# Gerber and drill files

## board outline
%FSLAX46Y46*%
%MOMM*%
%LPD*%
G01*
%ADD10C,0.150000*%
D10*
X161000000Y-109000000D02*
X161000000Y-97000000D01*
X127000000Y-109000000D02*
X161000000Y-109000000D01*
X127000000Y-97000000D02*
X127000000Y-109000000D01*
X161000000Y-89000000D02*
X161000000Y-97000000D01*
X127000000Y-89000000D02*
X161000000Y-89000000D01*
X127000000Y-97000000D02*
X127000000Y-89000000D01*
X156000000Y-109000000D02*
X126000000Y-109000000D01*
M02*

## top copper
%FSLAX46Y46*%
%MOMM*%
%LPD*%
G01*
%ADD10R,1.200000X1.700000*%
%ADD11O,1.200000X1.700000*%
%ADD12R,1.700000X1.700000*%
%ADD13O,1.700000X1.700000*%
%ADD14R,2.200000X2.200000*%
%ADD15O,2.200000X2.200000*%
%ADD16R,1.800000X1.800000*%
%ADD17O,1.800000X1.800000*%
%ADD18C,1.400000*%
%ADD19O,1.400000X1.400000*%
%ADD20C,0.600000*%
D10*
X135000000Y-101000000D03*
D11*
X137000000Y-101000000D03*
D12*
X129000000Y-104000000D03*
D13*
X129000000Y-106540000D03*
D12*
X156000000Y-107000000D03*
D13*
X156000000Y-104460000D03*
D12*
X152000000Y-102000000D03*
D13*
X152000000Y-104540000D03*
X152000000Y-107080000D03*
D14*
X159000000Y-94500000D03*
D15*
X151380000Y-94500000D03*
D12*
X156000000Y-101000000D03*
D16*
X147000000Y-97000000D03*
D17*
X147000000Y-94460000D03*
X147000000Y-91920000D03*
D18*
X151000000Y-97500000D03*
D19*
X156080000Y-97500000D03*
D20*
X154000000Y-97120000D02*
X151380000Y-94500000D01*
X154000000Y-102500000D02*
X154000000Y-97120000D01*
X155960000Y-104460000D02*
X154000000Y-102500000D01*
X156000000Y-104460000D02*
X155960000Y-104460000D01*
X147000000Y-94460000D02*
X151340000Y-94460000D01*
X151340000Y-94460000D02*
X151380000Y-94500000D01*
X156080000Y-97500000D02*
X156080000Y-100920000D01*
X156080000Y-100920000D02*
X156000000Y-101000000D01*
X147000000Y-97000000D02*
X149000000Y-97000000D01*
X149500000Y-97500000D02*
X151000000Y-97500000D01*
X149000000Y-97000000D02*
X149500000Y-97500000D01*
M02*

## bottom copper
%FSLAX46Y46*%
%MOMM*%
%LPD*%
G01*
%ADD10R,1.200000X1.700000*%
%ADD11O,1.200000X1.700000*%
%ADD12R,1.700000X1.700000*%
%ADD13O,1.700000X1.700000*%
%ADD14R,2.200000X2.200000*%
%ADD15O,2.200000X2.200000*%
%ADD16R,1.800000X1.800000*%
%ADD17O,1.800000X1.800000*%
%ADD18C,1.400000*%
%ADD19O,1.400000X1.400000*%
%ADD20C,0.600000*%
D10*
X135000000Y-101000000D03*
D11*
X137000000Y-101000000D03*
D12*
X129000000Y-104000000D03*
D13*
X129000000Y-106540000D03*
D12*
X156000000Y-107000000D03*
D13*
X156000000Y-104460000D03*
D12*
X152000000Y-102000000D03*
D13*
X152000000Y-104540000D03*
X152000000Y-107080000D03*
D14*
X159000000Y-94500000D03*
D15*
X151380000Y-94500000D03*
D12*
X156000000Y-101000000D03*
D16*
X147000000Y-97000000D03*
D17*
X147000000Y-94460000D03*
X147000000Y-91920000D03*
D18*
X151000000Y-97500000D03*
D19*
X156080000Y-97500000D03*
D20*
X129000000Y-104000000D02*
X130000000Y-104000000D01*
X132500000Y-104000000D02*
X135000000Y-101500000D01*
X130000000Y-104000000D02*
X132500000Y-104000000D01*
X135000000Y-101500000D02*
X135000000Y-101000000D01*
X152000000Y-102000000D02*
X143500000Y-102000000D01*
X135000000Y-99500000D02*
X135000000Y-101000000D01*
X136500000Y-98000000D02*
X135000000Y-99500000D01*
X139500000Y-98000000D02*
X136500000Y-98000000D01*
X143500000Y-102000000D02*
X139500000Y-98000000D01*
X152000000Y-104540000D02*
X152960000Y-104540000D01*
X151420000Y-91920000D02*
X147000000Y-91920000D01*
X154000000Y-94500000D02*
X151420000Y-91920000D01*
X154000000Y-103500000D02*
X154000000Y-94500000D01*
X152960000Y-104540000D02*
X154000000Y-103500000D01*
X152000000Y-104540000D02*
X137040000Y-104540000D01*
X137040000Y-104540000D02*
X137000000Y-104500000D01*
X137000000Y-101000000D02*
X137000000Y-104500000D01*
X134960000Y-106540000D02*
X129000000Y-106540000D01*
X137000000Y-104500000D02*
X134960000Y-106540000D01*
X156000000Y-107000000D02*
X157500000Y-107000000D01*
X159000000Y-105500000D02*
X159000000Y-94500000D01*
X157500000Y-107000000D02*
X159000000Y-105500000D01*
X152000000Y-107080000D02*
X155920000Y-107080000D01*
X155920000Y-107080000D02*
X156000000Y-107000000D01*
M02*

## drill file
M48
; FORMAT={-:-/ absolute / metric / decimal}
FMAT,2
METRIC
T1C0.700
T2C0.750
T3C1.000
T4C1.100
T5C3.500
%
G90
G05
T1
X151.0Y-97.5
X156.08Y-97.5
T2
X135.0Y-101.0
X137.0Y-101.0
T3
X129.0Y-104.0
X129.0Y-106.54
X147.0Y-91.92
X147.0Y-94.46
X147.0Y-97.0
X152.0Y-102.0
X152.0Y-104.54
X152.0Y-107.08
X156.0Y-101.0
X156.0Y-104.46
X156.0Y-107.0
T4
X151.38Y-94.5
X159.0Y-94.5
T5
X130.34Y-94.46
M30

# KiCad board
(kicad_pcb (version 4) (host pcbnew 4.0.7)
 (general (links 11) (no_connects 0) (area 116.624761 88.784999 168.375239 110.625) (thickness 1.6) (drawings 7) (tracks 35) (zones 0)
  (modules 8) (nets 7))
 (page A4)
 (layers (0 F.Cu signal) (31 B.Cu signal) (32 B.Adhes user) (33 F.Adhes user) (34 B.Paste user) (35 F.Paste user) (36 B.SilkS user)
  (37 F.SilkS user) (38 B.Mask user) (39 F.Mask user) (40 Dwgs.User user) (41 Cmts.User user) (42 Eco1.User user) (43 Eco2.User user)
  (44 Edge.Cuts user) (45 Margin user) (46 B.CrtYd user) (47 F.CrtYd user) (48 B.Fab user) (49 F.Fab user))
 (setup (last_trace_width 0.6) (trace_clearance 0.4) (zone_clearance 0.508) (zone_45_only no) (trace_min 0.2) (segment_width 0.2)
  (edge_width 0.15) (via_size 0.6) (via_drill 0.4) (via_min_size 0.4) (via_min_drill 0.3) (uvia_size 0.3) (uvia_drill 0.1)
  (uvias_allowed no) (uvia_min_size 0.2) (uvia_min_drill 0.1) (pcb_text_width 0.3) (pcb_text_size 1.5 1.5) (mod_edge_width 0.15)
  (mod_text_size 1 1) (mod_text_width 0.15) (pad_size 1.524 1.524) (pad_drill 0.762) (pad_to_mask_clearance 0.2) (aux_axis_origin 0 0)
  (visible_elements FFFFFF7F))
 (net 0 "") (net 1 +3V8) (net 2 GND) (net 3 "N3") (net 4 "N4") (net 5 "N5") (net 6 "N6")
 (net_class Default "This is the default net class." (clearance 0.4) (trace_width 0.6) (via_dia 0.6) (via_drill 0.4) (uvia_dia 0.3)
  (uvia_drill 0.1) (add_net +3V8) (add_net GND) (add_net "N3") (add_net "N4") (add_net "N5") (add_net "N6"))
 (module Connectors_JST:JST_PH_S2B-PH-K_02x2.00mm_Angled (layer F.Cu) (at 135 101)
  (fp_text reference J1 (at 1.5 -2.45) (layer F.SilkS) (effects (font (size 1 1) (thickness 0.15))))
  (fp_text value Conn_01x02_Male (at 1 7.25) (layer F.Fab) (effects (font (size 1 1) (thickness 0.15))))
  (pad 1 thru_hole rect (at 0 0) (size 1.2 1.7) (drill 0.75) (layers *.Cu *.Mask) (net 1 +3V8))
  (pad 2 thru_hole oval (at 2 0) (size 1.2 1.7) (drill 0.75) (layers *.Cu *.Mask) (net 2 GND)))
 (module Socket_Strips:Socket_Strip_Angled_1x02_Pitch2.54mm (layer F.Cu) (at 129 104)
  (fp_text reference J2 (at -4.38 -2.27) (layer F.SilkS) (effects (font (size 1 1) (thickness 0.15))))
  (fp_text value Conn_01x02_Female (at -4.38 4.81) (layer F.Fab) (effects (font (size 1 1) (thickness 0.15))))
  (pad 1 thru_hole rect (at 0 0) (size 1.7 1.7) (drill 1) (layers *.Cu *.Mask) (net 1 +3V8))
  (pad 2 thru_hole oval (at 0 2.54) (size 1.7 1.7) (drill 1) (layers *.Cu *.Mask) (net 2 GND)))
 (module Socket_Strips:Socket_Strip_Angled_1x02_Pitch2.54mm (layer F.Cu) (at 156 107 180)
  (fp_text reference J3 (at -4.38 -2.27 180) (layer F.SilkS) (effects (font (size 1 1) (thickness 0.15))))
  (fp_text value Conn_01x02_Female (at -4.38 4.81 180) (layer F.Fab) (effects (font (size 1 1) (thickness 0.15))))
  (pad 1 thru_hole rect (at 0 0 180) (size 1.7 1.7) (drill 1) (layers *.Cu *.Mask) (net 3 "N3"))
  (pad 2 thru_hole oval (at 0 2.54 180) (size 1.7 1.7) (drill 1) (layers *.Cu *.Mask) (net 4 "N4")))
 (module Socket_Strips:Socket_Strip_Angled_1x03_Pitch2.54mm (layer F.Cu) (at 152 102)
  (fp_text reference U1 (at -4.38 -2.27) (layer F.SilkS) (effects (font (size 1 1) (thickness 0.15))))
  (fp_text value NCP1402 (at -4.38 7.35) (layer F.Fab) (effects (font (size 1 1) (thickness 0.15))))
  (pad 1 thru_hole rect (at 0 0) (size 1.7 1.7) (drill 1) (layers *.Cu *.Mask) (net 1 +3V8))
  (pad 2 thru_hole oval (at 0 2.54) (size 1.7 1.7) (drill 1) (layers *.Cu *.Mask) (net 2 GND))
  (pad 3 thru_hole oval (at 0 5.08) (size 1.7 1.7) (drill 1) (layers *.Cu *.Mask) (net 3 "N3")))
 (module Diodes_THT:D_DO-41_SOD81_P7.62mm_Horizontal (layer F.Cu) (at 159 94.5 180)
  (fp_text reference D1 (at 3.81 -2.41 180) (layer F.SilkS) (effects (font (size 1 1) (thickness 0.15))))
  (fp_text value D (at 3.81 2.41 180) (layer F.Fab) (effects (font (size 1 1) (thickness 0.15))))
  (pad 1 thru_hole rect (at 0 0 180) (size 2.2 2.2) (drill 1.1) (layers *.Cu *.Mask) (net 3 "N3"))
  (pad 2 thru_hole oval (at 7.62 0 180) (size 2.2 2.2) (drill 1.1) (layers *.Cu *.Mask) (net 4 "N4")))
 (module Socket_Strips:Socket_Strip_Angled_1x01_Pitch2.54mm (layer F.Cu) (at 156 101 180)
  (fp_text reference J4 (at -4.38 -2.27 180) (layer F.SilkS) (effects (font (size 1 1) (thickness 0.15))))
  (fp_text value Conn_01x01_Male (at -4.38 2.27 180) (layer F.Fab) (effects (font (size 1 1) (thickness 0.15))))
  (pad 1 thru_hole rect (at 0 0 180) (size 1.7 1.7) (drill 1) (layers *.Cu *.Mask) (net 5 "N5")))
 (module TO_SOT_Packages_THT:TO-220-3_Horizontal (layer F.Cu) (at 147 97 90)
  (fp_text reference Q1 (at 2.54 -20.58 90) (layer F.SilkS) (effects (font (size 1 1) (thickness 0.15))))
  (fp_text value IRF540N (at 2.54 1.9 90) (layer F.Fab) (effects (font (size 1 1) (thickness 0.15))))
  (pad 0 np_thru_hole oval (at 2.54 -16.66 90) (size 3.5 3.5) (drill 3.5) (layers *.Cu *.Mask))
  (pad 1 thru_hole rect (at 0 0 90) (size 1.8 1.8) (drill 1) (layers *.Cu *.Mask) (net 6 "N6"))
  (pad 2 thru_hole oval (at 2.54 0 90) (size 1.8 1.8) (drill 1) (layers *.Cu *.Mask) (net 4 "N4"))
  (pad 3 thru_hole oval (at 5.08 0 90) (size 1.8 1.8) (drill 1) (layers *.Cu *.Mask) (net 2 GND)))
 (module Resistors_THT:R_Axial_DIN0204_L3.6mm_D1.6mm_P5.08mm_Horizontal (layer F.Cu) (at 151 97.5)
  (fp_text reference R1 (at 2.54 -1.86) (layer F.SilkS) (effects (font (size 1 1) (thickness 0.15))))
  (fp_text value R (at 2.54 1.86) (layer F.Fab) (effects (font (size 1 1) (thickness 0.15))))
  (pad 1 thru_hole circle (at 0 0) (size 1.4 1.4) (drill 0.7) (layers *.Cu *.Mask) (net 6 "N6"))
  (pad 2 thru_hole oval (at 5.08 0) (size 1.4 1.4) (drill 0.7) (layers *.Cu *.Mask) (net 5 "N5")))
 (gr_line (start 161 109) (end 161 97) (angle 90) (layer Edge.Cuts) (width 0.15))
 (gr_line (start 127 109) (end 161 109) (angle 90) (layer Edge.Cuts) (width 0.15))
 (gr_line (start 127 97) (end 127 109) (angle 90) (layer Edge.Cuts) (width 0.15))
 (gr_line (start 161 89) (end 161 97) (angle 90) (layer Edge.Cuts) (width 0.15))
 (gr_line (start 127 89) (end 161 89) (angle 90) (layer Edge.Cuts) (width 0.15))
 (gr_line (start 127 97) (end 127 89) (angle 90) (layer Edge.Cuts) (width 0.15))
 (gr_line (start 156 109) (end 126 109) (angle 90) (layer Edge.Cuts) (width 0.15))
 (segment (start 129 104) (end 130 104) (width 0.6) (layer B.Cu) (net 1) (status 400000))
 (segment (start 132.5 104) (end 135 101.5) (width 0.6) (layer B.Cu) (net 1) (status 800000))
 (segment (start 130 104) (end 132.5 104) (width 0.6) (layer B.Cu) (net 1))
 (segment (start 135 101.5) (end 135 101) (width 0.6) (layer B.Cu) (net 1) (status C00000))
 (segment (start 152 102) (end 143.5 102) (width 0.6) (layer B.Cu) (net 1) (status 400000))
 (segment (start 135 99.5) (end 135 101) (width 0.6) (layer B.Cu) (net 1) (status 800000))
 (segment (start 136.5 98) (end 135 99.5) (width 0.6) (layer B.Cu) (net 1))
 (segment (start 139.5 98) (end 136.5 98) (width 0.6) (layer B.Cu) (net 1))
 (segment (start 143.5 102) (end 139.5 98) (width 0.6) (layer B.Cu) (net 1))
 (segment (start 152 104.54) (end 152.96 104.54) (width 0.6) (layer B.Cu) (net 2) (status 400000))
 (segment (start 151.42 91.92) (end 147 91.92) (width 0.6) (layer B.Cu) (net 2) (status 800000))
 (segment (start 154 94.5) (end 151.42 91.92) (width 0.6) (layer B.Cu) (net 2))
 (segment (start 154 103.5) (end 154 94.5) (width 0.6) (layer B.Cu) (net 2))
 (segment (start 152.96 104.54) (end 154 103.5) (width 0.6) (layer B.Cu) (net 2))
 (segment (start 152 104.54) (end 137.04 104.54) (width 0.6) (layer B.Cu) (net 2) (status 400000))
 (segment (start 137.04 104.54) (end 137 104.5) (width 0.6) (layer B.Cu) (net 2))
 (segment (start 137 101) (end 137 104.5) (width 0.6) (layer B.Cu) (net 2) (status 400000))
 (segment (start 134.96 106.54) (end 129 106.54) (width 0.6) (layer B.Cu) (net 2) (status 800000))
 (segment (start 137 104.5) (end 134.96 106.54) (width 0.6) (layer B.Cu) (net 2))
 (segment (start 156 107) (end 157.5 107) (width 0.6) (layer B.Cu) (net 3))
 (segment (start 159 105.5) (end 159 94.5) (width 0.6) (layer B.Cu) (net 3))
 (segment (start 157.5 107) (end 159 105.5) (width 0.6) (layer B.Cu) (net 3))
 (segment (start 152 107.08) (end 155.92 107.08) (width 0.6) (layer B.Cu) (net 3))
 (segment (start 155.92 107.08) (end 156 107) (width 0.6) (layer B.Cu) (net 3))
 (segment (start 154 97.12) (end 151.38 94.5) (width 0.6) (layer F.Cu) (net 4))
 (segment (start 154 102.5) (end 154 97.12) (width 0.6) (layer F.Cu) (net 4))
 (segment (start 155.96 104.46) (end 154 102.5) (width 0.6) (layer F.Cu) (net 4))
 (segment (start 156 104.46) (end 155.96 104.46) (width 0.6) (layer F.Cu) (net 4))
 (segment (start 147 94.46) (end 151.34 94.46) (width 0.6) (layer F.Cu) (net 4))
 (segment (start 151.34 94.46) (end 151.38 94.5) (width 0.6) (layer F.Cu) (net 4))
 (segment (start 156.08 97.5) (end 156.08 100.92) (width 0.6) (layer F.Cu) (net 5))
 (segment (start 156.08 100.92) (end 156 101) (width 0.6) (layer F.Cu) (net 5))
 (segment (start 147 97) (end 149 97) (width 0.6) (layer F.Cu) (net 6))
 (segment (start 149.5 97.5) (end 151 97.5) (width 0.6) (layer F.Cu) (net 6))
 (segment (start 149 97) (end 149.5 97.5) (width 0.6) (layer F.Cu) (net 6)))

